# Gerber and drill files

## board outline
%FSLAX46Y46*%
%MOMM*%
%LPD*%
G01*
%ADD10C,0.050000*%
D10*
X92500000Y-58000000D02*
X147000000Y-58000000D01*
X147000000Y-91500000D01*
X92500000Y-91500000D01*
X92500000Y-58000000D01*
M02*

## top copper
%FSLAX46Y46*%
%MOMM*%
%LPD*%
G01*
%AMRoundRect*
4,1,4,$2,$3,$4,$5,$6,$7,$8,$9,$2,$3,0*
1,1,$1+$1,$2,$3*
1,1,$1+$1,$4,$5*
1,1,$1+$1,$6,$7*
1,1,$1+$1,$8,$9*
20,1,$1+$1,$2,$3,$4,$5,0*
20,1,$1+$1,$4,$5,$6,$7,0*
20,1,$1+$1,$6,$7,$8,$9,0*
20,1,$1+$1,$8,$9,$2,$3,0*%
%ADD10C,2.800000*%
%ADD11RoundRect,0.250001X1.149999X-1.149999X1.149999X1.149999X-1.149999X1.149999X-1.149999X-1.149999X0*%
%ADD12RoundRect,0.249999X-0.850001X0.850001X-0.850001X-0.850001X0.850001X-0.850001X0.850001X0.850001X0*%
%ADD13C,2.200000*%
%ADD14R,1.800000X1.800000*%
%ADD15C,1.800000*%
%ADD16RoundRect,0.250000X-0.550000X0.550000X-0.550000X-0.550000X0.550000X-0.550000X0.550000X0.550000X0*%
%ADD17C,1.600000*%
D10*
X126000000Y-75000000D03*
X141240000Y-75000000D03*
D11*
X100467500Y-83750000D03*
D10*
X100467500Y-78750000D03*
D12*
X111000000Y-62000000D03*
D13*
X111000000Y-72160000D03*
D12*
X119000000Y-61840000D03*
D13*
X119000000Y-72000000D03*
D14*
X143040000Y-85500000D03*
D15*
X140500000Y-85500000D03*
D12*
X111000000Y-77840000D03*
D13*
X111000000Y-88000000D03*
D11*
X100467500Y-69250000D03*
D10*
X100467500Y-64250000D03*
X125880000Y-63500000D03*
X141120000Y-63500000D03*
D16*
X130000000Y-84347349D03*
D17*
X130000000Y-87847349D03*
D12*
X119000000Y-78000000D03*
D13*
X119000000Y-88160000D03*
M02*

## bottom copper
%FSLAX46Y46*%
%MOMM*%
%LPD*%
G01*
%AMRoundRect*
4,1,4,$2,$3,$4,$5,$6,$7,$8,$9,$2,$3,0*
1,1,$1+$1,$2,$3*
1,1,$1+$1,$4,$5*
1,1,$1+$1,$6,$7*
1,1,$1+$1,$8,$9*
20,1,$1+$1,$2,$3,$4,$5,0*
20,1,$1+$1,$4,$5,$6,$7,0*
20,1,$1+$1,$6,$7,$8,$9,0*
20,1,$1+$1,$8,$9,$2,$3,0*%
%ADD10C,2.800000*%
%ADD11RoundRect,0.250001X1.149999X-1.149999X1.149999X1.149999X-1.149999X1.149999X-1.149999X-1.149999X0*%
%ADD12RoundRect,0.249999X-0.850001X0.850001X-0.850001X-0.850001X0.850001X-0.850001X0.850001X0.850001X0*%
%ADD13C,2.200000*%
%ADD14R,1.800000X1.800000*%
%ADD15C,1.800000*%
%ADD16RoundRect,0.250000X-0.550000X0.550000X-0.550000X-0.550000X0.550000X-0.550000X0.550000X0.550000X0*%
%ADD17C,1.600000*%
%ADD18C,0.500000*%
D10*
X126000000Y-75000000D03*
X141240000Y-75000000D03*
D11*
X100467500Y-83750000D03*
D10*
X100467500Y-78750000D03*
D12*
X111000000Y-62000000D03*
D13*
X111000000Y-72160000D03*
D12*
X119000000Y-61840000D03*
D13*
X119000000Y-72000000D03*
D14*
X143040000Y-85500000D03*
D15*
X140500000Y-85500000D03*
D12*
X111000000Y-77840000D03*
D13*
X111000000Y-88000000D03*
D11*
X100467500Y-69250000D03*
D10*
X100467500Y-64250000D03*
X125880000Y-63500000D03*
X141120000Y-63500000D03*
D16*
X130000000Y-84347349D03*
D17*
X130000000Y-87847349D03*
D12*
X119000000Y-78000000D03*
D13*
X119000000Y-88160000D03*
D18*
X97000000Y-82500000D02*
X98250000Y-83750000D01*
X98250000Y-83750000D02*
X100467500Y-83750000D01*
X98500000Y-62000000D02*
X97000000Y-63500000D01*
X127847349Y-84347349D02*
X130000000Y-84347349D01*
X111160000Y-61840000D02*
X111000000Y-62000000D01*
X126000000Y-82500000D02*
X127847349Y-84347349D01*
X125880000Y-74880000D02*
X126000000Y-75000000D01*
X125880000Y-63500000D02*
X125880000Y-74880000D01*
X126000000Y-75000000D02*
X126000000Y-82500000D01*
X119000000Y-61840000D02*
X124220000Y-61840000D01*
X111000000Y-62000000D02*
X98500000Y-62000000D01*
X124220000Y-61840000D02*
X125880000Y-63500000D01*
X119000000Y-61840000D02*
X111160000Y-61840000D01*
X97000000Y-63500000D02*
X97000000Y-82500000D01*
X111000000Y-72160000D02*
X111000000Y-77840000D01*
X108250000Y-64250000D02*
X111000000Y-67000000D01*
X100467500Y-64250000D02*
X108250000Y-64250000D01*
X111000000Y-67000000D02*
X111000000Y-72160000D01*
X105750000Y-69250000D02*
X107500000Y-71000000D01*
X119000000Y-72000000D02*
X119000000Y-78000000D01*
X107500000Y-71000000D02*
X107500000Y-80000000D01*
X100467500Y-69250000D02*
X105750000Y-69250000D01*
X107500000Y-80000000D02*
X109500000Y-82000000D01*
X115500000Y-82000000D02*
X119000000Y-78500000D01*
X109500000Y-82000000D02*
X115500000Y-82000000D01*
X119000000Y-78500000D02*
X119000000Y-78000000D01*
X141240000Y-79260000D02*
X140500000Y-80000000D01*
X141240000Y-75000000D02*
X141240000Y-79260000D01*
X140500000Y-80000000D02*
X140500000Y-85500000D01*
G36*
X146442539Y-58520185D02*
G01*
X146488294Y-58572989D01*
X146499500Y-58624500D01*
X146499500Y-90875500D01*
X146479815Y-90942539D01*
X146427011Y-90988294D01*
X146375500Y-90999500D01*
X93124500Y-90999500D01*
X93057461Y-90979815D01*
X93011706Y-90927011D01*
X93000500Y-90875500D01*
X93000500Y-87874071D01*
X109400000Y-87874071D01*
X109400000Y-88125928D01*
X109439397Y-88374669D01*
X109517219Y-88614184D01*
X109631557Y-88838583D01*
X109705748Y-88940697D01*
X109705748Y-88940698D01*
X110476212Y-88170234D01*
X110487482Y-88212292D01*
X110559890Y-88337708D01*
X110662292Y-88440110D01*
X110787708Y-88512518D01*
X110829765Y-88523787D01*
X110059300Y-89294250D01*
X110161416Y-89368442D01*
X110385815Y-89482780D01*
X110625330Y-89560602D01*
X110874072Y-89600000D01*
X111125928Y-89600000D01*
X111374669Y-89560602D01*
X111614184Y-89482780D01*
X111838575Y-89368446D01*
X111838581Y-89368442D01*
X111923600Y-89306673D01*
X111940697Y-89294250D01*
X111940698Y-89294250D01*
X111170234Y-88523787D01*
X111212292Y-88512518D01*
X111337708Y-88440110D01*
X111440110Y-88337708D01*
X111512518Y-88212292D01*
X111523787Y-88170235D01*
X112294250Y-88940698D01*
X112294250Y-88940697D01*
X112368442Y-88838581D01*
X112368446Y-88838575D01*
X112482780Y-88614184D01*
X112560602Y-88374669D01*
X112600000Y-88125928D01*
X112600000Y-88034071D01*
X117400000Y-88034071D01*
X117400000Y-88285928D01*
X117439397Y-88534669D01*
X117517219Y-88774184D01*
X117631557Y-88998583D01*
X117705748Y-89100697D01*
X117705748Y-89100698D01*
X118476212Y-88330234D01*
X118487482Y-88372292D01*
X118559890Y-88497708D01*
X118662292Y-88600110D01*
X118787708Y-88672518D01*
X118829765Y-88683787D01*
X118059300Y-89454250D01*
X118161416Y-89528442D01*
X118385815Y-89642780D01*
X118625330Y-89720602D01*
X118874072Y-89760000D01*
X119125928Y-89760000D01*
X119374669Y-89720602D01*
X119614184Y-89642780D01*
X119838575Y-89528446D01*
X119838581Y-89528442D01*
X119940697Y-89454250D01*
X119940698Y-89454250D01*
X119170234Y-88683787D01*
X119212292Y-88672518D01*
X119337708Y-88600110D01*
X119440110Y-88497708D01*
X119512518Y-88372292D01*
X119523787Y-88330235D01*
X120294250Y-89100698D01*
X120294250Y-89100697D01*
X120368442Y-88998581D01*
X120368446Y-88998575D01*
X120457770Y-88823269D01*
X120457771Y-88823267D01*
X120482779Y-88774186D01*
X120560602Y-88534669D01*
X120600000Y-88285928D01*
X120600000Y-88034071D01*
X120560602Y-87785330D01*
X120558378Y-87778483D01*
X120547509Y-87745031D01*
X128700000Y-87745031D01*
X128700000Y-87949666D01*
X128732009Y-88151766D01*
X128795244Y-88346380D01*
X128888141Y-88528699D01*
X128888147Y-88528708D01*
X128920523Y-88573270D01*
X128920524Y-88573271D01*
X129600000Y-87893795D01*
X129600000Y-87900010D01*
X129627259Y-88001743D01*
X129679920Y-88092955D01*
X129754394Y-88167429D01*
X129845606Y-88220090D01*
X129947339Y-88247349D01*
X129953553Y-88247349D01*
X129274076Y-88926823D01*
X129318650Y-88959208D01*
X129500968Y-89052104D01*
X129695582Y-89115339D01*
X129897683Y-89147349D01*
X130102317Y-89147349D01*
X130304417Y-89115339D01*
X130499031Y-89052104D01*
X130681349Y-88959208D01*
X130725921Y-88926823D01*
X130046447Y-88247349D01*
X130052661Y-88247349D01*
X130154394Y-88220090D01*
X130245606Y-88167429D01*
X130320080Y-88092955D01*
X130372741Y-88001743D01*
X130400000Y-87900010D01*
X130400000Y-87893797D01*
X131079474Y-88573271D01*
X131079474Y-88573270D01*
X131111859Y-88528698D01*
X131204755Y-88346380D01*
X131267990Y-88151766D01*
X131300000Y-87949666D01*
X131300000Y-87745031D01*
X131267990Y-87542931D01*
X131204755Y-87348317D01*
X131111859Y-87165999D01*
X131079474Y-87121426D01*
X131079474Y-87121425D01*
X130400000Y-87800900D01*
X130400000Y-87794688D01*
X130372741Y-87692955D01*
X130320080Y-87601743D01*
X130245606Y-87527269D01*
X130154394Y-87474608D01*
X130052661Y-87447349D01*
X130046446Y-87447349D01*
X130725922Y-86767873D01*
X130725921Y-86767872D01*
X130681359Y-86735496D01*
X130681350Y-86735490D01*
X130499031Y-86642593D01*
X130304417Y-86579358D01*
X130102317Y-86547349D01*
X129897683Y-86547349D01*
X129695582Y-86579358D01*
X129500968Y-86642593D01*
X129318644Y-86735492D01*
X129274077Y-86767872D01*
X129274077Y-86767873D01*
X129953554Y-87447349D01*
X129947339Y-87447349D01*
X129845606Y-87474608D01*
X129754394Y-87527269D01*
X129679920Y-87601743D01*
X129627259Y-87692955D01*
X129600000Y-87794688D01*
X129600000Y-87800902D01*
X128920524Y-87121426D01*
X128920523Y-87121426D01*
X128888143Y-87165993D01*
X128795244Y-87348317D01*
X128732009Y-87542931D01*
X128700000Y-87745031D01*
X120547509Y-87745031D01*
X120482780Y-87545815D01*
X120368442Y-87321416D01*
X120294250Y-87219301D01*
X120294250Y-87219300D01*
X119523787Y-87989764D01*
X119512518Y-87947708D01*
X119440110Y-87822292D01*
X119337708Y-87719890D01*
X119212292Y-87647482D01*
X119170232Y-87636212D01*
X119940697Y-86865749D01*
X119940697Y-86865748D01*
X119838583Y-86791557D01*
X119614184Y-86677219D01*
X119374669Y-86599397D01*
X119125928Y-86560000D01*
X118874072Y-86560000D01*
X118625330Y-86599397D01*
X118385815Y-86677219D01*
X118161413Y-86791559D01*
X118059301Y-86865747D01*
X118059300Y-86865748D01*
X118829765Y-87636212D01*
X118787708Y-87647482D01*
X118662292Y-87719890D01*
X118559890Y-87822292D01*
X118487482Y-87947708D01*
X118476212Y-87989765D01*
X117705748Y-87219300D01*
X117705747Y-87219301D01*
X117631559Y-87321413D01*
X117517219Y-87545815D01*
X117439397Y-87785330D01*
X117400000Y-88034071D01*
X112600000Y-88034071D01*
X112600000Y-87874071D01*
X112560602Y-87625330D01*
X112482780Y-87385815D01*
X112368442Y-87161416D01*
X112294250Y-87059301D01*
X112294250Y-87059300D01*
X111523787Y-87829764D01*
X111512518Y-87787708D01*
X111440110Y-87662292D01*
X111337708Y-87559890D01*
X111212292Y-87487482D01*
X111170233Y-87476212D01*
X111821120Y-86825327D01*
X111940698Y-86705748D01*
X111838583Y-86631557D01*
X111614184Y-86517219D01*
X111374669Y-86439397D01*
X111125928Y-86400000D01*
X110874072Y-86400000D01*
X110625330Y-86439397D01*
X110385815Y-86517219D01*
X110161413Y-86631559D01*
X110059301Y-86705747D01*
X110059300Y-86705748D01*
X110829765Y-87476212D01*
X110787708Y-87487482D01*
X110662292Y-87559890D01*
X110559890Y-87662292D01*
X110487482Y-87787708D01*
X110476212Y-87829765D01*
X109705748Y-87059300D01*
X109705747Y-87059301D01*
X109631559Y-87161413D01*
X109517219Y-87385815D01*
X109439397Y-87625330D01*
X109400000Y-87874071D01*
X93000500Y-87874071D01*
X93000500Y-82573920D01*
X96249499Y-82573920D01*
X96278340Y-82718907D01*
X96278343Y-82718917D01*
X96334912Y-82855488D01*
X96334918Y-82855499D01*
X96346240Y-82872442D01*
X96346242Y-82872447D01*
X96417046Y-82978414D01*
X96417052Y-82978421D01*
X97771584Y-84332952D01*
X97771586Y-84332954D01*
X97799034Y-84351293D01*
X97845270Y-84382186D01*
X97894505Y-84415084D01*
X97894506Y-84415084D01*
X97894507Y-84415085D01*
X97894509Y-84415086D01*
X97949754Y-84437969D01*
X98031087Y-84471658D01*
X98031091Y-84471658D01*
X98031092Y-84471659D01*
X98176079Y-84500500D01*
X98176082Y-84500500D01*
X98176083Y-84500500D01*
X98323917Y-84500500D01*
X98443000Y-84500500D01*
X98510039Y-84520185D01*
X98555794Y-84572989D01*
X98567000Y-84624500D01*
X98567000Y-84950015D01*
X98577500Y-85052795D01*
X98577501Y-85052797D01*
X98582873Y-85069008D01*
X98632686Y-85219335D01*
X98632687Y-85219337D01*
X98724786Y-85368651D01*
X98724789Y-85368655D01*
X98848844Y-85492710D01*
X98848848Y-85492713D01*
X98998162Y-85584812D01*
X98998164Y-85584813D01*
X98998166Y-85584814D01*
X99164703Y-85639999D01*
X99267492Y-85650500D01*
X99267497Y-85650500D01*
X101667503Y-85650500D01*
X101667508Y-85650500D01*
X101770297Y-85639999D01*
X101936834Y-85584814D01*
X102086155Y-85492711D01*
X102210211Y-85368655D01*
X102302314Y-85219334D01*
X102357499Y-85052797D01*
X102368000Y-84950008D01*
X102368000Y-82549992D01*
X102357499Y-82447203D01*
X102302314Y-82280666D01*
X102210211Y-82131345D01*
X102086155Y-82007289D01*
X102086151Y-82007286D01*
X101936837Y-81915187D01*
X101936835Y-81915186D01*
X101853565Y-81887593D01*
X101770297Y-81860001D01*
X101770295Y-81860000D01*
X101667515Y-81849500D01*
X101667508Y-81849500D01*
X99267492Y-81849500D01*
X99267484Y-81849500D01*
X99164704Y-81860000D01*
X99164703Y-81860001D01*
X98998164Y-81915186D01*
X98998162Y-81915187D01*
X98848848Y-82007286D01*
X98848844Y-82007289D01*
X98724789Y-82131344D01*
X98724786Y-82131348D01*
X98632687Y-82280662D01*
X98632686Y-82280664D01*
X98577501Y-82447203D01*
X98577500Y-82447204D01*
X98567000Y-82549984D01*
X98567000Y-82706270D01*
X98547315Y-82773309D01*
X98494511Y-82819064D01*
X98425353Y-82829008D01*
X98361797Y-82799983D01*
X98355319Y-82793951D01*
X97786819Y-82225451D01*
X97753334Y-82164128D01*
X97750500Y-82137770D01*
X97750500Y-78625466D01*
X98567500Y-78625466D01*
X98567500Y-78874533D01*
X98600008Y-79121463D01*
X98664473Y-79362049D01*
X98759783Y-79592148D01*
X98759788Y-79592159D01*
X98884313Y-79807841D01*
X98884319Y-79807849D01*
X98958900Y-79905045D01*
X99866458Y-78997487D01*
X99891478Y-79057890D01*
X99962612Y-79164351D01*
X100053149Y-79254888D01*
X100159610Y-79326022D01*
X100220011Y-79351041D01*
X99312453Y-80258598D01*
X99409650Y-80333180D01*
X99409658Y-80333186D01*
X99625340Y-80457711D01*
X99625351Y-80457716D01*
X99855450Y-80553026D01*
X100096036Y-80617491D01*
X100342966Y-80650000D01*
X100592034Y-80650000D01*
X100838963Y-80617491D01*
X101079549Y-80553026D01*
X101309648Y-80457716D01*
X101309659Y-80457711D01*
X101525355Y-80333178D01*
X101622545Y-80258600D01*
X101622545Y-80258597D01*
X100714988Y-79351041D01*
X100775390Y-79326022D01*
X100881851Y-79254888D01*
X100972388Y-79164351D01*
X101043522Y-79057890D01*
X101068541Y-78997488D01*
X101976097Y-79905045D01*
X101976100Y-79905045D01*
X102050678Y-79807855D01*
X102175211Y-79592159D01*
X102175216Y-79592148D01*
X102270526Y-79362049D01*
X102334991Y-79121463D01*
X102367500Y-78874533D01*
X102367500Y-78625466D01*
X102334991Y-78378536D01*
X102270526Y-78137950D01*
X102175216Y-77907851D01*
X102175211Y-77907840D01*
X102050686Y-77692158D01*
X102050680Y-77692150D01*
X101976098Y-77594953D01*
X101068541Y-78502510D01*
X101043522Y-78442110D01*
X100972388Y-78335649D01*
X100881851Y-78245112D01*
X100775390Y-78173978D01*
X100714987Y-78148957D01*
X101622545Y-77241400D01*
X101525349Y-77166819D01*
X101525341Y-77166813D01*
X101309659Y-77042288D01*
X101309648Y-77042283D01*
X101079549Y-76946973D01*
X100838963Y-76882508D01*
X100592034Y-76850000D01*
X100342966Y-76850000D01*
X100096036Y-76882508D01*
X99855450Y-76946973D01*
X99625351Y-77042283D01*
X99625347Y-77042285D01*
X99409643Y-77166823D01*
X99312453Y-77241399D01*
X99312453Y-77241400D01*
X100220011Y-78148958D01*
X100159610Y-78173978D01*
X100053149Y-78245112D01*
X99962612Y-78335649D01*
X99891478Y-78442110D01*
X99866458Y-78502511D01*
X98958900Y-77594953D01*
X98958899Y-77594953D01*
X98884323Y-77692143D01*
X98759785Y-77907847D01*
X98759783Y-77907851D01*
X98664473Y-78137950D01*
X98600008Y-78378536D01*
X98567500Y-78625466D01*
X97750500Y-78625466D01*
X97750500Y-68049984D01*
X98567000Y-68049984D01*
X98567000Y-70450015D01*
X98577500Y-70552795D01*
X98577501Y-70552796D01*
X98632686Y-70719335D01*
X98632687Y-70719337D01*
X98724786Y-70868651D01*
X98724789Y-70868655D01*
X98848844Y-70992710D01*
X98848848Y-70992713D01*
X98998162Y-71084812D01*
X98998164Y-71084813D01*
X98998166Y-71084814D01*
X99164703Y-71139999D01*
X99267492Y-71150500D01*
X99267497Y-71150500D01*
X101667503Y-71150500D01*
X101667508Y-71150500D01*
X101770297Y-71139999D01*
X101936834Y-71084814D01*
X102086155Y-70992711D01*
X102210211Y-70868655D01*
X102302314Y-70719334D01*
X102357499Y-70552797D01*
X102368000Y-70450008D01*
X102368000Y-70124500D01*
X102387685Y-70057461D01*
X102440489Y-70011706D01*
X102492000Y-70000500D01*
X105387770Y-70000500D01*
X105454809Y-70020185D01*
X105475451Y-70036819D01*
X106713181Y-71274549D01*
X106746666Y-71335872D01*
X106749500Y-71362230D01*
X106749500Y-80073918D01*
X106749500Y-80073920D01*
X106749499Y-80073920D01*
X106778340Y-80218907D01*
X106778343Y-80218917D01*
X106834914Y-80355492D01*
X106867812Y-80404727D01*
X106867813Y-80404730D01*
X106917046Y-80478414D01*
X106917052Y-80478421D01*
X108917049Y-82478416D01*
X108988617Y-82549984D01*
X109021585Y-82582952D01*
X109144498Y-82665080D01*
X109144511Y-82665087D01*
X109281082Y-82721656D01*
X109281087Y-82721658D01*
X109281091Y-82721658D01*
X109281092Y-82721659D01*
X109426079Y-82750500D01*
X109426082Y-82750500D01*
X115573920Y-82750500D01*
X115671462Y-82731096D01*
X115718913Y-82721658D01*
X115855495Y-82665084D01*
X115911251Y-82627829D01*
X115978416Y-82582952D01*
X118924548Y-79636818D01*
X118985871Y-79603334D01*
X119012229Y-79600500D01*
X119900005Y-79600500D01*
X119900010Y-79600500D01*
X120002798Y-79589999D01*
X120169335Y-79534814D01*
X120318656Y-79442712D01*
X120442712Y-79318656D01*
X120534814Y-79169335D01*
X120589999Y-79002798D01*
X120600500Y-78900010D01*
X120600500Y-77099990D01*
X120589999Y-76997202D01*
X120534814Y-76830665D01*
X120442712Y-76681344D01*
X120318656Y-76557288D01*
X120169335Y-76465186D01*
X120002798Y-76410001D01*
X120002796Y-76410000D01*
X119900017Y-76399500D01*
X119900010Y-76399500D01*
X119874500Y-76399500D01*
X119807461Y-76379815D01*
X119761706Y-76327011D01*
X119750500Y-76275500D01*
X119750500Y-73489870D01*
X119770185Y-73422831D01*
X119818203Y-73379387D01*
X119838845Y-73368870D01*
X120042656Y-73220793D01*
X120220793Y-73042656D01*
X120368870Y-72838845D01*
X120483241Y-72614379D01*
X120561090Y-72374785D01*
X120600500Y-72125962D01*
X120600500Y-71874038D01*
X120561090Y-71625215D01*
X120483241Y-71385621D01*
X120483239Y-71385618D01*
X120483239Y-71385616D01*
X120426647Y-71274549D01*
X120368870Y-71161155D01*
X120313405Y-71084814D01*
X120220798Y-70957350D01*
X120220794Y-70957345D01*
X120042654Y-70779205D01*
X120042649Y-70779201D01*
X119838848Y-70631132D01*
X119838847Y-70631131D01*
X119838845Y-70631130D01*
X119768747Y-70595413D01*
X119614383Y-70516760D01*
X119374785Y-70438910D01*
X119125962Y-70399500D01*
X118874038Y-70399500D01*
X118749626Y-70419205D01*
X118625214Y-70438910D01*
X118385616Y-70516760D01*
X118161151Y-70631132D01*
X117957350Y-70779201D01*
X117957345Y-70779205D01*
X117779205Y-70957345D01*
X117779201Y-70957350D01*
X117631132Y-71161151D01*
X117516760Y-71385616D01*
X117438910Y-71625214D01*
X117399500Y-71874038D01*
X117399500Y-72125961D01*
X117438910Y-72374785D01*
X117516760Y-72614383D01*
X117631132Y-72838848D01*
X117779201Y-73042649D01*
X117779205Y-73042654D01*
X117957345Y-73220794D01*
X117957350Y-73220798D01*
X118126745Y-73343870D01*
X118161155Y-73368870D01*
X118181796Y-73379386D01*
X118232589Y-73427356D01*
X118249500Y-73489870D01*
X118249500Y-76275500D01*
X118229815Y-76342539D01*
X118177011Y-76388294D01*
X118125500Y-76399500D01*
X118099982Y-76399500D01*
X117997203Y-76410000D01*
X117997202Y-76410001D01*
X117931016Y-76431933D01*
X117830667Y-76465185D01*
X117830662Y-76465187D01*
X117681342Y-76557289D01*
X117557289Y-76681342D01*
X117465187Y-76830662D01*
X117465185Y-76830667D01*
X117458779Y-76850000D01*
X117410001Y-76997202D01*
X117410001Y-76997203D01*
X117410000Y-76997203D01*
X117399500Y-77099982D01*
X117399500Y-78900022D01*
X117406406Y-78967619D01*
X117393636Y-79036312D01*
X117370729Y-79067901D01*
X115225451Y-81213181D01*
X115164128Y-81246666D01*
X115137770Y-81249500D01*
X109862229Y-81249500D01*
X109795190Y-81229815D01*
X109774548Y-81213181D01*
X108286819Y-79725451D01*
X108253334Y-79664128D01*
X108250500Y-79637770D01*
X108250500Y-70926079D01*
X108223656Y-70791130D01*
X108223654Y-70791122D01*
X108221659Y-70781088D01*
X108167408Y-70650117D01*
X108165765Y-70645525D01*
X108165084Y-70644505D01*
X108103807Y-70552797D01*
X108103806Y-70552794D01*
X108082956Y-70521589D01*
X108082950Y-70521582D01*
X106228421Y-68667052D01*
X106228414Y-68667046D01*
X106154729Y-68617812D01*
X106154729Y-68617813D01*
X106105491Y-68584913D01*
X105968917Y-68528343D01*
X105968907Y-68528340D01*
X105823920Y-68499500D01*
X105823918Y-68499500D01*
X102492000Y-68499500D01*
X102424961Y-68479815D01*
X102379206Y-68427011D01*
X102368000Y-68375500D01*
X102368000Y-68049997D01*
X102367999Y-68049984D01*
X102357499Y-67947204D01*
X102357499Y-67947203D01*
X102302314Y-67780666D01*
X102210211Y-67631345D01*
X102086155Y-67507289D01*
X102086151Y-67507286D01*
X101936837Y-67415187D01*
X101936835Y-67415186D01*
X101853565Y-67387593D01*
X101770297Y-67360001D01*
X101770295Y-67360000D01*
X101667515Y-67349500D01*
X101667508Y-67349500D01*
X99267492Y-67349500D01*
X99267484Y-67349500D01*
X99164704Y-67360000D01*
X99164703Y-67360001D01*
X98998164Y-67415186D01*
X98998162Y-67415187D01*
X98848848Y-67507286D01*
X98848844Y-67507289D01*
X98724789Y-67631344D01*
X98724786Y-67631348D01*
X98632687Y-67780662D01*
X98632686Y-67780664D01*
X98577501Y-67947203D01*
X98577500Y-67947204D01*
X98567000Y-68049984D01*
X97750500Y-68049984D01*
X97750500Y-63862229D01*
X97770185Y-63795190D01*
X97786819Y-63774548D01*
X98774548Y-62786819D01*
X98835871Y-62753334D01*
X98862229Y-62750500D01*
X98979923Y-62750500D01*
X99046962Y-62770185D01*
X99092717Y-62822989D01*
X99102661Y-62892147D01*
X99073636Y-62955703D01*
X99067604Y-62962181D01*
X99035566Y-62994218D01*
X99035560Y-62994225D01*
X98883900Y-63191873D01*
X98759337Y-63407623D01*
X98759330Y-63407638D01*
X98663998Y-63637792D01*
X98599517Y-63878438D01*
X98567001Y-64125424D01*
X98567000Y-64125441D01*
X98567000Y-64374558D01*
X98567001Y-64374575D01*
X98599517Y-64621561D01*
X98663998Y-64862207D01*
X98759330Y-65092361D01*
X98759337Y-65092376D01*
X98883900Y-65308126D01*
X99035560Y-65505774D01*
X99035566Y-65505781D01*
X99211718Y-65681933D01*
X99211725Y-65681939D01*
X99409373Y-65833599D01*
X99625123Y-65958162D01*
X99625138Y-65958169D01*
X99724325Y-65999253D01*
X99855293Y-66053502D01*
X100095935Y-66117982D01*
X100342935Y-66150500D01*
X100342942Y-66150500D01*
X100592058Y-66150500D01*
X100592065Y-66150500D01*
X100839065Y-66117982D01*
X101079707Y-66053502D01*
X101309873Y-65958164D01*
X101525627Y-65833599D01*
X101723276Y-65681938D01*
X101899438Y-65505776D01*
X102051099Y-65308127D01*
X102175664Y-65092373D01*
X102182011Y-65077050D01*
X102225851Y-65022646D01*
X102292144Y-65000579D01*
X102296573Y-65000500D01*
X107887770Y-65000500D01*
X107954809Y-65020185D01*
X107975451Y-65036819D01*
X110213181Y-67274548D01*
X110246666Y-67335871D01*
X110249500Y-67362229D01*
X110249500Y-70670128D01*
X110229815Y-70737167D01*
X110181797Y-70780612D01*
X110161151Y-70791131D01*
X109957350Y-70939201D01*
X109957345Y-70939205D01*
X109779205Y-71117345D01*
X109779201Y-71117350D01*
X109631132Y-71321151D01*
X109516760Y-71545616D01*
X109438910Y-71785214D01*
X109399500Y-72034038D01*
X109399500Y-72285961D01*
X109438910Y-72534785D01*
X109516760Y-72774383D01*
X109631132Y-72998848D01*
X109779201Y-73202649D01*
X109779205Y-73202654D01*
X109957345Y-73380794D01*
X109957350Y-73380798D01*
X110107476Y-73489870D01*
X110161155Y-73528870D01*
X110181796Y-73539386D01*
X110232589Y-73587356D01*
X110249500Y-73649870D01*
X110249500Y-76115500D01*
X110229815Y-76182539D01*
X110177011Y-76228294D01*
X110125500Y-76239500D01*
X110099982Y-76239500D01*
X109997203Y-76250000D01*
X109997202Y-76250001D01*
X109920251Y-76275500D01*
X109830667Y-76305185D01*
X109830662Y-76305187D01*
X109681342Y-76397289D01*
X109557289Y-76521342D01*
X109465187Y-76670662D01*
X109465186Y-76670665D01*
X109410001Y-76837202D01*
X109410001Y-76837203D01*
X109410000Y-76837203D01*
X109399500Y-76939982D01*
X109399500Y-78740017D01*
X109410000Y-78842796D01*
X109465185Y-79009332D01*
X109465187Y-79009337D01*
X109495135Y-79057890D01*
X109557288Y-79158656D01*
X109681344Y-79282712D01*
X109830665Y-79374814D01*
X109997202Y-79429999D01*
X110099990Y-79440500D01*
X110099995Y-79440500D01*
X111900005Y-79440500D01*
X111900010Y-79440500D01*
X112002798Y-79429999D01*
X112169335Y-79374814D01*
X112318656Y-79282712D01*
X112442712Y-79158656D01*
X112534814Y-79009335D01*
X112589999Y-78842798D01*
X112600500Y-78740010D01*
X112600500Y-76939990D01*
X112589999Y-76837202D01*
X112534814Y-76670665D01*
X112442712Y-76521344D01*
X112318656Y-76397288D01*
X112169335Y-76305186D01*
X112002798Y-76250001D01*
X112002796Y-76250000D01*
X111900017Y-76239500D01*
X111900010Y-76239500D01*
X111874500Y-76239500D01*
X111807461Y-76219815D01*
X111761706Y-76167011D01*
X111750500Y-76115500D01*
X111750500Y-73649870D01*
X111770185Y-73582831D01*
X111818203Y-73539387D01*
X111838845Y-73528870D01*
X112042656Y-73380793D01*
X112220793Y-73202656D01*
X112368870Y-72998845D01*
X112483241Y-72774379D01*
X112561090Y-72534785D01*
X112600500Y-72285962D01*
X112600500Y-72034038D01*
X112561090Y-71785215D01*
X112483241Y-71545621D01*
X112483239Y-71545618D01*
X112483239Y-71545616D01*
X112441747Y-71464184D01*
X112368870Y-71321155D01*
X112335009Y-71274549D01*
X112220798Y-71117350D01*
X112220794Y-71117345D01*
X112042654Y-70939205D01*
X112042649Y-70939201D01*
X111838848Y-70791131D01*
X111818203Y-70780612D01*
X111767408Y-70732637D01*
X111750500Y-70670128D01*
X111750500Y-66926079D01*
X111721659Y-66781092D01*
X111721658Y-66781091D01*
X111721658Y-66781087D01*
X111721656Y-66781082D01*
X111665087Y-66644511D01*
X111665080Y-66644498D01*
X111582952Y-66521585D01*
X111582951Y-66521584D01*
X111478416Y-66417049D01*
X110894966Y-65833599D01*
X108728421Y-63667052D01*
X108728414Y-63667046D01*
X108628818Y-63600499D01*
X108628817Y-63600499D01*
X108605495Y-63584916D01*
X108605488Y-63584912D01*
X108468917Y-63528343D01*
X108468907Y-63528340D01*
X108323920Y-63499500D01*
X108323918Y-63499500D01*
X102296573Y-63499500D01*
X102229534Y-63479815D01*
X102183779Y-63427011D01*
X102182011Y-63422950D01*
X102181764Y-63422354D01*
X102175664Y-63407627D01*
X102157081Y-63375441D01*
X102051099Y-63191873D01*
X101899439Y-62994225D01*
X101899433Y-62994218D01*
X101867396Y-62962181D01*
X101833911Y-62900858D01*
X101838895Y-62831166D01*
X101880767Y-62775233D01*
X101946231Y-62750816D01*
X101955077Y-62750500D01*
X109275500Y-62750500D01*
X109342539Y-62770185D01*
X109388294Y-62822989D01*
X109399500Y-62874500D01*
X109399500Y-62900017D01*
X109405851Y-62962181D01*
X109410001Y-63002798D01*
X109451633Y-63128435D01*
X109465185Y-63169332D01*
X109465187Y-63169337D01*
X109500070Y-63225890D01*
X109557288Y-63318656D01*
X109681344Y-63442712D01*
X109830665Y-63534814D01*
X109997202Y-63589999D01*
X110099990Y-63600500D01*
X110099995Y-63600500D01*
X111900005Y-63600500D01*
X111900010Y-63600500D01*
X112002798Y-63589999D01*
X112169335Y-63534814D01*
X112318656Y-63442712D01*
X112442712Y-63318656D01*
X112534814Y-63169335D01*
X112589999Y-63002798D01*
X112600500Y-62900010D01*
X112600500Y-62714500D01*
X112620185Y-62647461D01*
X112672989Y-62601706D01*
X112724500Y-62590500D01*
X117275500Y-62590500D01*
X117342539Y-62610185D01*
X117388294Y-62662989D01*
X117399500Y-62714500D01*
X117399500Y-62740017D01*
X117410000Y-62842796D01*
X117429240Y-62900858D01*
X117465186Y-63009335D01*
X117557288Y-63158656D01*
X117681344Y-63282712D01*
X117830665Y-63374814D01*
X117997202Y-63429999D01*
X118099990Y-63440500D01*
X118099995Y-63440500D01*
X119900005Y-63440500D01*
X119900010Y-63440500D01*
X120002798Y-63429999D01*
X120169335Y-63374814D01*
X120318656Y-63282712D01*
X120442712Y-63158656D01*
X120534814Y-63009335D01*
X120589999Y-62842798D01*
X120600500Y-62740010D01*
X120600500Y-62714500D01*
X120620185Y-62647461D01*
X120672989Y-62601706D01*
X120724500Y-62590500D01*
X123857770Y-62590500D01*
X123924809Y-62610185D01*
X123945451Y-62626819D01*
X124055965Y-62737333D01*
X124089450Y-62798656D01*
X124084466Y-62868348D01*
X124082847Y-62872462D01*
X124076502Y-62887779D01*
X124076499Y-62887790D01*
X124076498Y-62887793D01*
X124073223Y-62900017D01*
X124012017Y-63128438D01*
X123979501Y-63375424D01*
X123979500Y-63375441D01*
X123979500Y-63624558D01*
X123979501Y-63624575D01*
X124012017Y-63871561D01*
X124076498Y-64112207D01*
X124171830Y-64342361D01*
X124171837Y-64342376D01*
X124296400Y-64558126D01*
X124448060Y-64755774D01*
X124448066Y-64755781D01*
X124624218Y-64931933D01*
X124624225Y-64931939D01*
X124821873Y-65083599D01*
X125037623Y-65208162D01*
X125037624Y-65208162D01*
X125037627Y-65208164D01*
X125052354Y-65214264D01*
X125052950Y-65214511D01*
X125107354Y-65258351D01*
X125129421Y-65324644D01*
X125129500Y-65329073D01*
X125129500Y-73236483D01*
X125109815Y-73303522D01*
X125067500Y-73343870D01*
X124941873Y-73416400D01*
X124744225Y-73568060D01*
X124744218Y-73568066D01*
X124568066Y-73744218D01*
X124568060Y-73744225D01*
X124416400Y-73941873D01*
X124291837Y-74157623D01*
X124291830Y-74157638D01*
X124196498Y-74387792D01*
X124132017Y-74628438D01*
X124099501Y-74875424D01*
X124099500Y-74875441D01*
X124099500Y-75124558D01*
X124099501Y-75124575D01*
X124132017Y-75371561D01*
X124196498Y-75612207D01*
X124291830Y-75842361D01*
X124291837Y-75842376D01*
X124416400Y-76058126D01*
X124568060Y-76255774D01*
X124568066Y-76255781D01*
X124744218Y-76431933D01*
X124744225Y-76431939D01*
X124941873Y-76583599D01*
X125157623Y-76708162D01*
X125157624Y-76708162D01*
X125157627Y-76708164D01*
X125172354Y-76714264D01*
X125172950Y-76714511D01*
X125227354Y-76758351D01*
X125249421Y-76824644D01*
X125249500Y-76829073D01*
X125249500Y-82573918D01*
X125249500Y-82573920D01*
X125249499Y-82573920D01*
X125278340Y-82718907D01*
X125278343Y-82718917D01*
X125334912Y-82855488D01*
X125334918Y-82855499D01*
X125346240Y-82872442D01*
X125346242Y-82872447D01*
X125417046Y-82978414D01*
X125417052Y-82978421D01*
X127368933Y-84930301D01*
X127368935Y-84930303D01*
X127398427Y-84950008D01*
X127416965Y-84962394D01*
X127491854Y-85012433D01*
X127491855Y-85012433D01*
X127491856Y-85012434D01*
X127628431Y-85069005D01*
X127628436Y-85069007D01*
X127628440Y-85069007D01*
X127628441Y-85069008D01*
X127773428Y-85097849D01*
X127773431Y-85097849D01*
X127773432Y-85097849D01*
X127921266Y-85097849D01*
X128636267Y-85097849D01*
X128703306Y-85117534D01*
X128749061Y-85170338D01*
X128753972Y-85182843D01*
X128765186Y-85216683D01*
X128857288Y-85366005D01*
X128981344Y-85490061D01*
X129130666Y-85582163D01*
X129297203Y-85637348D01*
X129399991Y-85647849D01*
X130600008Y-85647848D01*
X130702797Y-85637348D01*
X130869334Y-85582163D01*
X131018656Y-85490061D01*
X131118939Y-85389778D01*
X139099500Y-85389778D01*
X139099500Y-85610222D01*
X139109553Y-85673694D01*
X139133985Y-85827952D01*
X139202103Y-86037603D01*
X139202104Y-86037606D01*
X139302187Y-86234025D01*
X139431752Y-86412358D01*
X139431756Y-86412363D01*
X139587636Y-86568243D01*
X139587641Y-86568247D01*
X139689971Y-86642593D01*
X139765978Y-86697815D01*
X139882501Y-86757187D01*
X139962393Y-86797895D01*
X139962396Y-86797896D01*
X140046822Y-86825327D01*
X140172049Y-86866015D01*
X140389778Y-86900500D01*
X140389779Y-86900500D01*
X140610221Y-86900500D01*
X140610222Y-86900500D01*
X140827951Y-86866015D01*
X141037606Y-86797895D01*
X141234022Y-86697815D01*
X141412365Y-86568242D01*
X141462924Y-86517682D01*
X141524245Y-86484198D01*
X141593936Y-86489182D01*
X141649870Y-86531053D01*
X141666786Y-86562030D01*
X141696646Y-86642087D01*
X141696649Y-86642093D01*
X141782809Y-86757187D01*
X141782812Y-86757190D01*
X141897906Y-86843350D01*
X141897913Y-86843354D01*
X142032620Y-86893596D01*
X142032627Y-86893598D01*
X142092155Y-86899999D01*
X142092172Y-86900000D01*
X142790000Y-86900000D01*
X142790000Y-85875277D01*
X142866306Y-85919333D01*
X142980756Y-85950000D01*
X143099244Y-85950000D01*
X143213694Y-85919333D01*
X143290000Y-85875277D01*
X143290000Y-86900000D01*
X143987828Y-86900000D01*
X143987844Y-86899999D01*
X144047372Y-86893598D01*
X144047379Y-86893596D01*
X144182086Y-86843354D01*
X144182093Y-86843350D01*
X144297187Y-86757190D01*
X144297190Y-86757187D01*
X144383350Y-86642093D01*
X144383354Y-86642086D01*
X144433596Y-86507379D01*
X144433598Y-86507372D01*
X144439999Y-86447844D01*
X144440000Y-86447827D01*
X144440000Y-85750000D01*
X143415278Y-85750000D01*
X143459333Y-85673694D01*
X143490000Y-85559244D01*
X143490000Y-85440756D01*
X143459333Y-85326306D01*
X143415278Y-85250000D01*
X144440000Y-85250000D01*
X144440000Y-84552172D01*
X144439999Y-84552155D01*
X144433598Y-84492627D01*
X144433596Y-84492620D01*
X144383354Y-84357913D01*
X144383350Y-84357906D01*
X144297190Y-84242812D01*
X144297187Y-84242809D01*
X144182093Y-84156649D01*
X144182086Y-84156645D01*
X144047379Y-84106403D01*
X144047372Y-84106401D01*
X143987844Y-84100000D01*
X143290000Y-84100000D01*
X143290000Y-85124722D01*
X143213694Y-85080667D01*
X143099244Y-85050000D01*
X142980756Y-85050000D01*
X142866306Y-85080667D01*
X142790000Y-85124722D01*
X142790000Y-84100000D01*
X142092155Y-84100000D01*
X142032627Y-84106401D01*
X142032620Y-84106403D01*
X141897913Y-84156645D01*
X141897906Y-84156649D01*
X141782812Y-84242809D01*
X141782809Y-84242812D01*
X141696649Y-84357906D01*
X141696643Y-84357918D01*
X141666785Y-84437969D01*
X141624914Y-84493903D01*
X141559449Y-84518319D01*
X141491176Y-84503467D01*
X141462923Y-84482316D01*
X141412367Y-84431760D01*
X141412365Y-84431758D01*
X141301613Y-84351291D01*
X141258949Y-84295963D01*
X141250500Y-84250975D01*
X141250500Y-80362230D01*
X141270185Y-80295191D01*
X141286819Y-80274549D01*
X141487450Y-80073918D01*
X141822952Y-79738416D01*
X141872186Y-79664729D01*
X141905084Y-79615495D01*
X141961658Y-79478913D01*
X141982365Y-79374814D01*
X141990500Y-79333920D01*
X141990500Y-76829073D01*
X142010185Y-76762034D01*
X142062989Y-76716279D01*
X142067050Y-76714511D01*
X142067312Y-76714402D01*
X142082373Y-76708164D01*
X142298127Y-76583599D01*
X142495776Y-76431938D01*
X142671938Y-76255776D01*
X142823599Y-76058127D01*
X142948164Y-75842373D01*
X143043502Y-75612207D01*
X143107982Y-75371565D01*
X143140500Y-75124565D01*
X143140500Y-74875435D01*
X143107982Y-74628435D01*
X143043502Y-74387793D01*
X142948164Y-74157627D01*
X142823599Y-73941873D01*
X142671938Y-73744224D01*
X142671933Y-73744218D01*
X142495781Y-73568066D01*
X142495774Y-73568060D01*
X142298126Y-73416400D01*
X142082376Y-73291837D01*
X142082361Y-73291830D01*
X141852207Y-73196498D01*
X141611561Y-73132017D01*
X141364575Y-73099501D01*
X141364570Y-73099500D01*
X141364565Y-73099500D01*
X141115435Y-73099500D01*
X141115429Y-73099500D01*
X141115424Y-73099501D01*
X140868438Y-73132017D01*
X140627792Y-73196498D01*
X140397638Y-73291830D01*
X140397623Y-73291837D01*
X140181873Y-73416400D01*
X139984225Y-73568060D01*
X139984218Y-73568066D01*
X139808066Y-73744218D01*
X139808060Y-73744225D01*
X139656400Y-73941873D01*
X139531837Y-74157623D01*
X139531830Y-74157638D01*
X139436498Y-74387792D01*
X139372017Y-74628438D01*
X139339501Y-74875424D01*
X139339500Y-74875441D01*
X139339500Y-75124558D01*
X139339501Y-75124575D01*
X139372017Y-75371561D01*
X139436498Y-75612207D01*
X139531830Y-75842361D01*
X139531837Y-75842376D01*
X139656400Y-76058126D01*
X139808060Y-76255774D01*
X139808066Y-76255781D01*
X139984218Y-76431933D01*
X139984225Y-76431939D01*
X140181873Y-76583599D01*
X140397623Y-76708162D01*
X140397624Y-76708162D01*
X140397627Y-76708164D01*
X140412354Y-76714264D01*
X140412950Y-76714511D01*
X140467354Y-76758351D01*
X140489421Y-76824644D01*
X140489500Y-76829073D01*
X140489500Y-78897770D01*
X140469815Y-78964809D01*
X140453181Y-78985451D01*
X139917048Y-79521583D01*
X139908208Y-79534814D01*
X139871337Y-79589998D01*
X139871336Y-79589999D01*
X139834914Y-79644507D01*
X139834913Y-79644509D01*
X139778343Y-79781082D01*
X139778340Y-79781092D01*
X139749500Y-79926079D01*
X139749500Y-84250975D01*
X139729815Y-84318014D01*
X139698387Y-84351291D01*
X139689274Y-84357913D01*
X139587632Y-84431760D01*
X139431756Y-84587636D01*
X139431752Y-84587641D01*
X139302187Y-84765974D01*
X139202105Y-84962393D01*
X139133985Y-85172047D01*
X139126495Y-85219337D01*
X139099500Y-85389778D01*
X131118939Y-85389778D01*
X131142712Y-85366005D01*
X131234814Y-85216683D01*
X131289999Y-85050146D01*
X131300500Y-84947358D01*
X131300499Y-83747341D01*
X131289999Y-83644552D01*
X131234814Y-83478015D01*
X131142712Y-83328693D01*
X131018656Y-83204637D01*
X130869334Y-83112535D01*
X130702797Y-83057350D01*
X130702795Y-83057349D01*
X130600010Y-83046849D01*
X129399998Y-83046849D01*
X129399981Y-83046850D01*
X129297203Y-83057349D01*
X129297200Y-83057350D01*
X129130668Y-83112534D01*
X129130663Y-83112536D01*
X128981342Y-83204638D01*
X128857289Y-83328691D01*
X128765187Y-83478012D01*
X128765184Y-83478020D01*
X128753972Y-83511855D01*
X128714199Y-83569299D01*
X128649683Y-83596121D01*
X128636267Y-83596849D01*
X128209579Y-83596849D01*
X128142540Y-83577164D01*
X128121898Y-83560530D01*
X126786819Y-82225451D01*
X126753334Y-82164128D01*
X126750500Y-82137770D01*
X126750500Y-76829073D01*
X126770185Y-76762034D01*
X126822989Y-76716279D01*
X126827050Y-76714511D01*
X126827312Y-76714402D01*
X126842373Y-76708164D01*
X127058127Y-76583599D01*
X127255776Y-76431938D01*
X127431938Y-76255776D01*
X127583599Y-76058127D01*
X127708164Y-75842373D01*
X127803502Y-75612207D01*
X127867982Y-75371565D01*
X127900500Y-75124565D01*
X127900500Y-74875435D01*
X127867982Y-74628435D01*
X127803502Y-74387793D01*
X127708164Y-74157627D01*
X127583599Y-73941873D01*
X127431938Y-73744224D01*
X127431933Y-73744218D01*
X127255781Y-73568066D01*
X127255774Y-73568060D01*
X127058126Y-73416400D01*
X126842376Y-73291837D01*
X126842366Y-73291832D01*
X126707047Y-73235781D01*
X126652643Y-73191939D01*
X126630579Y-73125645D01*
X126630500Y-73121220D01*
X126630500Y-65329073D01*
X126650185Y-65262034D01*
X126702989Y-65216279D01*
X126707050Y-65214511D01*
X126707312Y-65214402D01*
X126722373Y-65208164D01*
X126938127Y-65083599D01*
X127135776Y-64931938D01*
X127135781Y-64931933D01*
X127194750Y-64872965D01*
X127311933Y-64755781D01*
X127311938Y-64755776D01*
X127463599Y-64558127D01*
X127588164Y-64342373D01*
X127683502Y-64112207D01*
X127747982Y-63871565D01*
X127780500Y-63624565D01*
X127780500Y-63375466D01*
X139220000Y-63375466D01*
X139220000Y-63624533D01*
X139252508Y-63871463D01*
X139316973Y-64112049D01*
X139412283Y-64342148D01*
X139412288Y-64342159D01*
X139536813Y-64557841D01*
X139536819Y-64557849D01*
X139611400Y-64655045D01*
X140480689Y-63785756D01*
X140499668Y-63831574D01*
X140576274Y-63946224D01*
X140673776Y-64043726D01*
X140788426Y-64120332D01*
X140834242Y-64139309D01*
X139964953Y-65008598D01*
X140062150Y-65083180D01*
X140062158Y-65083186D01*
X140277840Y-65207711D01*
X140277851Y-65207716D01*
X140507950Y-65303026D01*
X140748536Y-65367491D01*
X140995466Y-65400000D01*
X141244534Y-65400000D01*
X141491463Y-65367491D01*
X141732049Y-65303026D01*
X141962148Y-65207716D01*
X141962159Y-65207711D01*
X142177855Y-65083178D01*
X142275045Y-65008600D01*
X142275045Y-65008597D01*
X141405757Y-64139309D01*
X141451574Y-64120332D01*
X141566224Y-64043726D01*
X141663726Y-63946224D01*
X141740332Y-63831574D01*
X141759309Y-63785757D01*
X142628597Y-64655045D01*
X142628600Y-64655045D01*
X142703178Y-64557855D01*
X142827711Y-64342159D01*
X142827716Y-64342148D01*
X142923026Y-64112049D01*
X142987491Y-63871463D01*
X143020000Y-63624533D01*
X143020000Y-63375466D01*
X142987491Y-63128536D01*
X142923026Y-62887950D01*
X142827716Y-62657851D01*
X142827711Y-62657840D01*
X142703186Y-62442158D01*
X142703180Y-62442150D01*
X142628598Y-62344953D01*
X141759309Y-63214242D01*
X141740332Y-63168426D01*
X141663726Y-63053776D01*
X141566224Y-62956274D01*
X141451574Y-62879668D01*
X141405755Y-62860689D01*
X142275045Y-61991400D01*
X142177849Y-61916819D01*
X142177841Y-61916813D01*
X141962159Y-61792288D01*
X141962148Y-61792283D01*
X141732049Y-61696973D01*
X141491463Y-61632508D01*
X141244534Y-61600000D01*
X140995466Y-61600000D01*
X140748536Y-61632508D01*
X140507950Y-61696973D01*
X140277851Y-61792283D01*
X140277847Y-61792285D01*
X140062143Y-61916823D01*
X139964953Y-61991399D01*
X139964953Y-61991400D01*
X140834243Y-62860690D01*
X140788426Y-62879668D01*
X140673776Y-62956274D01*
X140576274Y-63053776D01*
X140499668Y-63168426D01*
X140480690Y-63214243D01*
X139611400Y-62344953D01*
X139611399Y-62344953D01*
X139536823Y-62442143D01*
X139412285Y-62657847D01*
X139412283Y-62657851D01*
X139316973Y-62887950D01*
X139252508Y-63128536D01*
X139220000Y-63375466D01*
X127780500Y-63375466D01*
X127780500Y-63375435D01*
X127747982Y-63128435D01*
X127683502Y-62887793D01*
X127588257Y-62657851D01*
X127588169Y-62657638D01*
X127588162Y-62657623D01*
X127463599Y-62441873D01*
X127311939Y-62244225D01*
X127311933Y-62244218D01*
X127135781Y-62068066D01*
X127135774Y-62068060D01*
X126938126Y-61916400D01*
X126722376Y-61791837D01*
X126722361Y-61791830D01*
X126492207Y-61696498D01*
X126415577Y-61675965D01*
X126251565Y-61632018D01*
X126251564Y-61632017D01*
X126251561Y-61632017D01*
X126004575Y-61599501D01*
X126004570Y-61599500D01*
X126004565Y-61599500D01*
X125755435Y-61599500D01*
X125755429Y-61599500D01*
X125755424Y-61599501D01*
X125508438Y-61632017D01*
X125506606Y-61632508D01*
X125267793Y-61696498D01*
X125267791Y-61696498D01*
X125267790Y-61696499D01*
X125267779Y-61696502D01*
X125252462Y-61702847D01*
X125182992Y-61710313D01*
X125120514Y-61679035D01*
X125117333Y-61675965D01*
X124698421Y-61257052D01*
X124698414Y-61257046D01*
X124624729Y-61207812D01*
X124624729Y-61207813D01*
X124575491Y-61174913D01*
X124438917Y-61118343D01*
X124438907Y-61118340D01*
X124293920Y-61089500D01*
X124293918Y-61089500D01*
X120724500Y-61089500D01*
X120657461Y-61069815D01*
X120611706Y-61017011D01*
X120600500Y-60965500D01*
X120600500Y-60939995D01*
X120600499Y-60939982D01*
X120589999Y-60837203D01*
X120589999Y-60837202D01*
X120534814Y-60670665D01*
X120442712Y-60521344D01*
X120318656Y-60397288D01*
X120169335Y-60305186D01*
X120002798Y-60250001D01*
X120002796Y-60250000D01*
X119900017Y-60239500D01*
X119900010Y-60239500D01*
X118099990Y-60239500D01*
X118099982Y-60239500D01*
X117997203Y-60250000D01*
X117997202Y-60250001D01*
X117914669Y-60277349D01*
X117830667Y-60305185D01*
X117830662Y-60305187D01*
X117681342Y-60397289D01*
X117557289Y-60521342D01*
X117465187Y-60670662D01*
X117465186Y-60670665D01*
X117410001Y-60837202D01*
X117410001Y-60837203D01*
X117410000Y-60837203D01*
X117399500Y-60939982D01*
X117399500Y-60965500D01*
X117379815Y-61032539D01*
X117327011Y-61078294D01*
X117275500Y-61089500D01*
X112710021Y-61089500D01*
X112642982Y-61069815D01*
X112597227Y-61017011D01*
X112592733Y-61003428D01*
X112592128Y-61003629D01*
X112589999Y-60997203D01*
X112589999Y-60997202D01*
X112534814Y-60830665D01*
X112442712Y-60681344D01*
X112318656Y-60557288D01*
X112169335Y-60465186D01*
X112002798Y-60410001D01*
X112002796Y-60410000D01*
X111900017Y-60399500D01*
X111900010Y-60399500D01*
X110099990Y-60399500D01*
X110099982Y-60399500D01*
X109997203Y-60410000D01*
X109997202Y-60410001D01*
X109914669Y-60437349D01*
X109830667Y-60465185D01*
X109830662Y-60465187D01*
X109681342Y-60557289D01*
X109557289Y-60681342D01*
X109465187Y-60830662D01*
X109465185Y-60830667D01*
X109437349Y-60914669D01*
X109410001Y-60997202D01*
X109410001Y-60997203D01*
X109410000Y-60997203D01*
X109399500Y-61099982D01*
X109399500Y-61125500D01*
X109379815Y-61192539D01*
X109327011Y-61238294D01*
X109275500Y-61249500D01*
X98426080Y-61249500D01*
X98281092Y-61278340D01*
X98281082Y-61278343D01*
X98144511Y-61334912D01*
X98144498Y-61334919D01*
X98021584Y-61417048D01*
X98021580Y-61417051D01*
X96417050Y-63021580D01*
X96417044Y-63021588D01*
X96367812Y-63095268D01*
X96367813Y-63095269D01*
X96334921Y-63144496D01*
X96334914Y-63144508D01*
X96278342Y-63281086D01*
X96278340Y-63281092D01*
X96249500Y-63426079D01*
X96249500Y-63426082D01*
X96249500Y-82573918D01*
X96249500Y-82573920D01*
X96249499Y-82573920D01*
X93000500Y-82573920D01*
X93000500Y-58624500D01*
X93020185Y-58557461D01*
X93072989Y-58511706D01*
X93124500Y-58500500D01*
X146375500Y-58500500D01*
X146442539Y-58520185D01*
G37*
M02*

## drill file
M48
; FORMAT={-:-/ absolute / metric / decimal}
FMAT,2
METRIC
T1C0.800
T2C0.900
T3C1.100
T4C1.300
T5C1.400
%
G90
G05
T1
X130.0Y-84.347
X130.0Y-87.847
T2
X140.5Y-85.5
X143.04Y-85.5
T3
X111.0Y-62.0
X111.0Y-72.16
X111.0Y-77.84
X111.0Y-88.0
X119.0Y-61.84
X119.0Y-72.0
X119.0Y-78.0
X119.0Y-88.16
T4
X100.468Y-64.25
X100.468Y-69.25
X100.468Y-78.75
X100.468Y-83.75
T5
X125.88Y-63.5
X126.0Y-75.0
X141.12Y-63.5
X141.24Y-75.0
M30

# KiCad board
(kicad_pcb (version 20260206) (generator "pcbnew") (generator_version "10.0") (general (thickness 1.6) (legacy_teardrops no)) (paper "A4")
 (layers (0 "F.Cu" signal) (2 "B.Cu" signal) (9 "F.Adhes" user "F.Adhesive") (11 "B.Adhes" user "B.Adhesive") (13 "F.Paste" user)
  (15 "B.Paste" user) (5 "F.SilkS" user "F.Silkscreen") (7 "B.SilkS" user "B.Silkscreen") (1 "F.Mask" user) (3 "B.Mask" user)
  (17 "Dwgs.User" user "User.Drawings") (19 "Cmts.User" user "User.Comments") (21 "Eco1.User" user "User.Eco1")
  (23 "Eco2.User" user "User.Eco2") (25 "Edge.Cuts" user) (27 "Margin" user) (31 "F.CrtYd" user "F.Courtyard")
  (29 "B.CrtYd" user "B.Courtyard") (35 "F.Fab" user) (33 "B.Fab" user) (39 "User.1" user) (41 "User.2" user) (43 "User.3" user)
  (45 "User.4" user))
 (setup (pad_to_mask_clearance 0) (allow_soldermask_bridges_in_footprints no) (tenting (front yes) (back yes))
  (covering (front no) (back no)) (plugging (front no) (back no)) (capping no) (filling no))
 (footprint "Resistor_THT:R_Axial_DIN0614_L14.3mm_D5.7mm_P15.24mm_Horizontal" (layer "F.Cu") (at 126 75)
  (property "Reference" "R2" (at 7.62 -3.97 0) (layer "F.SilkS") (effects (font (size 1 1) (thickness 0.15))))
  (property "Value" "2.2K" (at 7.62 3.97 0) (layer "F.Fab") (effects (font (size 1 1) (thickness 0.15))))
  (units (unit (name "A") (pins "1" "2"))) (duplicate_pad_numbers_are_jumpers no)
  (pad "1" thru_hole circle (at 0 0) (size 2.8 2.8) (drill 1.4) (layers "*.Cu" "*.Mask") (remove_unused_layers no) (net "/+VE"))
  (pad "2" thru_hole circle (at 15.24 0) (size 2.8 2.8) (drill 1.4) (layers "*.Cu" "*.Mask") (remove_unused_layers no) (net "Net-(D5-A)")))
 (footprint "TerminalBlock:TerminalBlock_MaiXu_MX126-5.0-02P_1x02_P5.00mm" (layer "F.Cu") (at 100.4675 83.75 90)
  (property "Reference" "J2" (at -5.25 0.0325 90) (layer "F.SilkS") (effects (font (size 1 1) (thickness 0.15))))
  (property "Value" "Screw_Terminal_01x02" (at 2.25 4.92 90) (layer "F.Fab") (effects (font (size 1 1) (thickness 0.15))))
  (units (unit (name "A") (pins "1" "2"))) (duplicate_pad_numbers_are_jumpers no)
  (pad "1" thru_hole roundrect (at 0 0 90) (size 2.8 2.8) (drill 1.3) (layers "*.Cu" "*.Mask") (remove_unused_layers no)
   (roundrect_rratio 0.089286) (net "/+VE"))
  (pad "2" thru_hole circle (at 5 0 90) (size 2.8 2.8) (drill 1.3) (layers "*.Cu" "*.Mask") (remove_unused_layers no) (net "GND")))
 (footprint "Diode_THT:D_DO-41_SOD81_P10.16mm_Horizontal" (layer "F.Cu") (at 111 62 -90)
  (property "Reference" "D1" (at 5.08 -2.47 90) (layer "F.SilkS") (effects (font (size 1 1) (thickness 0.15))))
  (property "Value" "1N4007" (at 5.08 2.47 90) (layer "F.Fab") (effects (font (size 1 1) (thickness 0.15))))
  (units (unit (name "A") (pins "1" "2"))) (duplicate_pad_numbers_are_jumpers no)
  (pad "1" thru_hole roundrect (at 0 0 270) (size 2.2 2.2) (drill 1.1) (layers "*.Cu" "*.Mask") (remove_unused_layers no)
   (roundrect_rratio 0.113636) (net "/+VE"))
  (pad "2" thru_hole circle (at 10.16 0 270) (size 2.2 2.2) (drill 1.1) (layers "*.Cu" "*.Mask") (remove_unused_layers no)
   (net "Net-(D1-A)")))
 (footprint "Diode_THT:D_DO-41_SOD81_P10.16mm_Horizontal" (layer "F.Cu") (at 119 61.84 -90)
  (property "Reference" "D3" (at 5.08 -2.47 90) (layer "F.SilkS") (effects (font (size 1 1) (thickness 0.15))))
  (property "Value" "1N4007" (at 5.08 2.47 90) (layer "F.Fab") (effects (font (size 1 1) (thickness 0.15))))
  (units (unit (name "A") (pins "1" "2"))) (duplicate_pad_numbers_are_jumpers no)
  (pad "1" thru_hole roundrect (at 0 0 270) (size 2.2 2.2) (drill 1.1) (layers "*.Cu" "*.Mask") (remove_unused_layers no)
   (roundrect_rratio 0.113636) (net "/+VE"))
  (pad "2" thru_hole circle (at 10.16 0 270) (size 2.2 2.2) (drill 1.1) (layers "*.Cu" "*.Mask") (remove_unused_layers no)
   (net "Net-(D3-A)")))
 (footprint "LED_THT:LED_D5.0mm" (layer "F.Cu") (at 143.04 85.5 180)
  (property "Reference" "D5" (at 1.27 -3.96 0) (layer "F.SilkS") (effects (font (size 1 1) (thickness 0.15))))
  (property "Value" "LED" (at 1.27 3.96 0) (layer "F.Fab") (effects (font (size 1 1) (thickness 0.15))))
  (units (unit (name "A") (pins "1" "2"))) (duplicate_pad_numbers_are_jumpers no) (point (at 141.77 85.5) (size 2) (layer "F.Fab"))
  (pad "1" thru_hole rect (at 0 0 180) (size 1.8 1.8) (drill 0.9) (layers "*.Cu" "*.Mask") (remove_unused_layers no) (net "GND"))
  (pad "2" thru_hole circle (at 2.54 0 180) (size 1.8 1.8) (drill 0.9) (layers "*.Cu" "*.Mask") (remove_unused_layers no) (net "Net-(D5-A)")))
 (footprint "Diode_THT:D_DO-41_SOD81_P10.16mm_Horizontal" (layer "F.Cu") (at 111 77.84 -90)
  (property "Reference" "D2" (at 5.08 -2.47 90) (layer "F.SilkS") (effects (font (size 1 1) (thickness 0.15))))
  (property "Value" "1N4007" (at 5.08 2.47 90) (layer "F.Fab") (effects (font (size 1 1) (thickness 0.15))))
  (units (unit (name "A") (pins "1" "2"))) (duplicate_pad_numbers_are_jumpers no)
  (pad "1" thru_hole roundrect (at 0 0 270) (size 2.2 2.2) (drill 1.1) (layers "*.Cu" "*.Mask") (remove_unused_layers no)
   (roundrect_rratio 0.113636) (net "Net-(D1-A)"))
  (pad "2" thru_hole circle (at 10.16 0 270) (size 2.2 2.2) (drill 1.1) (layers "*.Cu" "*.Mask") (remove_unused_layers no) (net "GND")))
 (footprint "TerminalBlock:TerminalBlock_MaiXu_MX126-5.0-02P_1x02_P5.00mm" (layer "F.Cu") (at 100.4675 69.25 90)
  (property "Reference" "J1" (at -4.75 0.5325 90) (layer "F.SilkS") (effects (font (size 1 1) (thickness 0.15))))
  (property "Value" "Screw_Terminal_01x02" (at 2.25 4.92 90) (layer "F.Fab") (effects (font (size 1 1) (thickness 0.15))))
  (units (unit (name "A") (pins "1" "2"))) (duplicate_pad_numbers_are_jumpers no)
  (pad "1" thru_hole roundrect (at 0 0 90) (size 2.8 2.8) (drill 1.3) (layers "*.Cu" "*.Mask") (remove_unused_layers no)
   (roundrect_rratio 0.089286) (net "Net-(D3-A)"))
  (pad "2" thru_hole circle (at 5 0 90) (size 2.8 2.8) (drill 1.3) (layers "*.Cu" "*.Mask") (remove_unused_layers no) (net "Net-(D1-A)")))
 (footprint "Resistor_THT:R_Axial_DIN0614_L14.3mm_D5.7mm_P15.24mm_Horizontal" (layer "F.Cu") (at 125.88 63.5)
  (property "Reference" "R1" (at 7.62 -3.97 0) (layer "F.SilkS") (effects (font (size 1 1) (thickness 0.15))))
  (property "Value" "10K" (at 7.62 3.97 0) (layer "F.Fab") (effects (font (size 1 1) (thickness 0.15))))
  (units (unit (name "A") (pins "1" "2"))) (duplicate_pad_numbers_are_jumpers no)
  (pad "1" thru_hole circle (at 0 0) (size 2.8 2.8) (drill 1.4) (layers "*.Cu" "*.Mask") (remove_unused_layers no) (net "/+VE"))
  (pad "2" thru_hole circle (at 15.24 0) (size 2.8 2.8) (drill 1.4) (layers "*.Cu" "*.Mask") (remove_unused_layers no) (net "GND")))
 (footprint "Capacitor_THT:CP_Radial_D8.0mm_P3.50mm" (layer "F.Cu") (at 130 84.347349 -90)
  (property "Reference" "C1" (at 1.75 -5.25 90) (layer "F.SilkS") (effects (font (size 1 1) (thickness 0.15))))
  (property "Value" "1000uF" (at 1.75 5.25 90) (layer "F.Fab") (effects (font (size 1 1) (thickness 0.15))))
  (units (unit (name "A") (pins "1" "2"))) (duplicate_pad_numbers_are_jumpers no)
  (pad "1" thru_hole roundrect (at 0 0 270) (size 1.6 1.6) (drill 0.8) (layers "*.Cu" "*.Mask") (remove_unused_layers no)
   (roundrect_rratio 0.15625) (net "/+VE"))
  (pad "2" thru_hole circle (at 3.5 0 270) (size 1.6 1.6) (drill 0.8) (layers "*.Cu" "*.Mask") (remove_unused_layers no) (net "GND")))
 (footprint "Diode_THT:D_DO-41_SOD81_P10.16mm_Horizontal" (layer "F.Cu") (at 119 78 -90)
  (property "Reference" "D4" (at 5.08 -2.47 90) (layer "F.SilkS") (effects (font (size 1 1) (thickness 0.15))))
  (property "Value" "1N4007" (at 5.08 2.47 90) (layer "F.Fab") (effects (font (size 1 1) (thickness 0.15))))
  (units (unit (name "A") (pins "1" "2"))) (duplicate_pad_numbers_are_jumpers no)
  (pad "1" thru_hole roundrect (at 0 0 270) (size 2.2 2.2) (drill 1.1) (layers "*.Cu" "*.Mask") (remove_unused_layers no)
   (roundrect_rratio 0.113636) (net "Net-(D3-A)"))
  (pad "2" thru_hole circle (at 10.16 0 270) (size 2.2 2.2) (drill 1.1) (layers "*.Cu" "*.Mask") (remove_unused_layers no) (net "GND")))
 (gr_rect (start 92.5 58) (end 147 91.5) (stroke (width 0.05) (type default)) (fill no) (layer "Edge.Cuts"))
 (segment (start 97 82.5) (end 98.25 83.75) (width 0.5) (layer "B.Cu") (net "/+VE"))
 (segment (start 98.25 83.75) (end 100.4675 83.75) (width 0.5) (layer "B.Cu") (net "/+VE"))
 (segment (start 98.5 62) (end 97 63.5) (width 0.5) (layer "B.Cu") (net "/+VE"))
 (segment (start 127.847349 84.347349) (end 130 84.347349) (width 0.5) (layer "B.Cu") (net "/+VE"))
 (segment (start 111.16 61.84) (end 111 62) (width 0.5) (layer "B.Cu") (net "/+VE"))
 (segment (start 126 82.5) (end 127.847349 84.347349) (width 0.5) (layer "B.Cu") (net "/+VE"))
 (segment (start 125.88 74.88) (end 126 75) (width 0.5) (layer "B.Cu") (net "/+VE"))
 (segment (start 125.88 63.5) (end 125.88 74.88) (width 0.5) (layer "B.Cu") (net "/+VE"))
 (segment (start 126 75) (end 126 82.5) (width 0.5) (layer "B.Cu") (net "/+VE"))
 (segment (start 119 61.84) (end 124.22 61.84) (width 0.5) (layer "B.Cu") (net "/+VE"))
 (segment (start 111 62) (end 98.5 62) (width 0.5) (layer "B.Cu") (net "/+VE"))
 (segment (start 124.22 61.84) (end 125.88 63.5) (width 0.5) (layer "B.Cu") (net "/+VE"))
 (segment (start 119 61.84) (end 111.16 61.84) (width 0.5) (layer "B.Cu") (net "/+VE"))
 (segment (start 97 63.5) (end 97 82.5) (width 0.5) (layer "B.Cu") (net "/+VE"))
 (segment (start 111 72.16) (end 111 77.84) (width 0.5) (layer "B.Cu") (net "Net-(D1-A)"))
 (segment (start 108.25 64.25) (end 111 67) (width 0.5) (layer "B.Cu") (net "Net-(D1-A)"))
 (segment (start 100.4675 64.25) (end 108.25 64.25) (width 0.5) (layer "B.Cu") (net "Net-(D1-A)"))
 (segment (start 111 67) (end 111 72.16) (width 0.5) (layer "B.Cu") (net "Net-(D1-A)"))
 (segment (start 105.75 69.25) (end 107.5 71) (width 0.5) (layer "B.Cu") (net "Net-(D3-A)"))
 (segment (start 119 72) (end 119 78) (width 0.5) (layer "B.Cu") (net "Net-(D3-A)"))
 (segment (start 107.5 71) (end 107.5 80) (width 0.5) (layer "B.Cu") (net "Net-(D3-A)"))
 (segment (start 100.4675 69.25) (end 105.75 69.25) (width 0.5) (layer "B.Cu") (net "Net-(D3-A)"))
 (segment (start 107.5 80) (end 109.5 82) (width 0.5) (layer "B.Cu") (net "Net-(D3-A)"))
 (segment (start 115.5 82) (end 119 78.5) (width 0.5) (layer "B.Cu") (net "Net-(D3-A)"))
 (segment (start 109.5 82) (end 115.5 82) (width 0.5) (layer "B.Cu") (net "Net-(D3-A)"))
 (segment (start 119 78.5) (end 119 78) (width 0.5) (layer "B.Cu") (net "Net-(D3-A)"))
 (segment (start 141.24 79.26) (end 140.5 80) (width 0.5) (layer "B.Cu") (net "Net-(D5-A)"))
 (segment (start 141.24 75) (end 141.24 79.26) (width 0.5) (layer "B.Cu") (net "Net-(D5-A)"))
 (segment (start 140.5 80) (end 140.5 85.5) (width 0.5) (layer "B.Cu") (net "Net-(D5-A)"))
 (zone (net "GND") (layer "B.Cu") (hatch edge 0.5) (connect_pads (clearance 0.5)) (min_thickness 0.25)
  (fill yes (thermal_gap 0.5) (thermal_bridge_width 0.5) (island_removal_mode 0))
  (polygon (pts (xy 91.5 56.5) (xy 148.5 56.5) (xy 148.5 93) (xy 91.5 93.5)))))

